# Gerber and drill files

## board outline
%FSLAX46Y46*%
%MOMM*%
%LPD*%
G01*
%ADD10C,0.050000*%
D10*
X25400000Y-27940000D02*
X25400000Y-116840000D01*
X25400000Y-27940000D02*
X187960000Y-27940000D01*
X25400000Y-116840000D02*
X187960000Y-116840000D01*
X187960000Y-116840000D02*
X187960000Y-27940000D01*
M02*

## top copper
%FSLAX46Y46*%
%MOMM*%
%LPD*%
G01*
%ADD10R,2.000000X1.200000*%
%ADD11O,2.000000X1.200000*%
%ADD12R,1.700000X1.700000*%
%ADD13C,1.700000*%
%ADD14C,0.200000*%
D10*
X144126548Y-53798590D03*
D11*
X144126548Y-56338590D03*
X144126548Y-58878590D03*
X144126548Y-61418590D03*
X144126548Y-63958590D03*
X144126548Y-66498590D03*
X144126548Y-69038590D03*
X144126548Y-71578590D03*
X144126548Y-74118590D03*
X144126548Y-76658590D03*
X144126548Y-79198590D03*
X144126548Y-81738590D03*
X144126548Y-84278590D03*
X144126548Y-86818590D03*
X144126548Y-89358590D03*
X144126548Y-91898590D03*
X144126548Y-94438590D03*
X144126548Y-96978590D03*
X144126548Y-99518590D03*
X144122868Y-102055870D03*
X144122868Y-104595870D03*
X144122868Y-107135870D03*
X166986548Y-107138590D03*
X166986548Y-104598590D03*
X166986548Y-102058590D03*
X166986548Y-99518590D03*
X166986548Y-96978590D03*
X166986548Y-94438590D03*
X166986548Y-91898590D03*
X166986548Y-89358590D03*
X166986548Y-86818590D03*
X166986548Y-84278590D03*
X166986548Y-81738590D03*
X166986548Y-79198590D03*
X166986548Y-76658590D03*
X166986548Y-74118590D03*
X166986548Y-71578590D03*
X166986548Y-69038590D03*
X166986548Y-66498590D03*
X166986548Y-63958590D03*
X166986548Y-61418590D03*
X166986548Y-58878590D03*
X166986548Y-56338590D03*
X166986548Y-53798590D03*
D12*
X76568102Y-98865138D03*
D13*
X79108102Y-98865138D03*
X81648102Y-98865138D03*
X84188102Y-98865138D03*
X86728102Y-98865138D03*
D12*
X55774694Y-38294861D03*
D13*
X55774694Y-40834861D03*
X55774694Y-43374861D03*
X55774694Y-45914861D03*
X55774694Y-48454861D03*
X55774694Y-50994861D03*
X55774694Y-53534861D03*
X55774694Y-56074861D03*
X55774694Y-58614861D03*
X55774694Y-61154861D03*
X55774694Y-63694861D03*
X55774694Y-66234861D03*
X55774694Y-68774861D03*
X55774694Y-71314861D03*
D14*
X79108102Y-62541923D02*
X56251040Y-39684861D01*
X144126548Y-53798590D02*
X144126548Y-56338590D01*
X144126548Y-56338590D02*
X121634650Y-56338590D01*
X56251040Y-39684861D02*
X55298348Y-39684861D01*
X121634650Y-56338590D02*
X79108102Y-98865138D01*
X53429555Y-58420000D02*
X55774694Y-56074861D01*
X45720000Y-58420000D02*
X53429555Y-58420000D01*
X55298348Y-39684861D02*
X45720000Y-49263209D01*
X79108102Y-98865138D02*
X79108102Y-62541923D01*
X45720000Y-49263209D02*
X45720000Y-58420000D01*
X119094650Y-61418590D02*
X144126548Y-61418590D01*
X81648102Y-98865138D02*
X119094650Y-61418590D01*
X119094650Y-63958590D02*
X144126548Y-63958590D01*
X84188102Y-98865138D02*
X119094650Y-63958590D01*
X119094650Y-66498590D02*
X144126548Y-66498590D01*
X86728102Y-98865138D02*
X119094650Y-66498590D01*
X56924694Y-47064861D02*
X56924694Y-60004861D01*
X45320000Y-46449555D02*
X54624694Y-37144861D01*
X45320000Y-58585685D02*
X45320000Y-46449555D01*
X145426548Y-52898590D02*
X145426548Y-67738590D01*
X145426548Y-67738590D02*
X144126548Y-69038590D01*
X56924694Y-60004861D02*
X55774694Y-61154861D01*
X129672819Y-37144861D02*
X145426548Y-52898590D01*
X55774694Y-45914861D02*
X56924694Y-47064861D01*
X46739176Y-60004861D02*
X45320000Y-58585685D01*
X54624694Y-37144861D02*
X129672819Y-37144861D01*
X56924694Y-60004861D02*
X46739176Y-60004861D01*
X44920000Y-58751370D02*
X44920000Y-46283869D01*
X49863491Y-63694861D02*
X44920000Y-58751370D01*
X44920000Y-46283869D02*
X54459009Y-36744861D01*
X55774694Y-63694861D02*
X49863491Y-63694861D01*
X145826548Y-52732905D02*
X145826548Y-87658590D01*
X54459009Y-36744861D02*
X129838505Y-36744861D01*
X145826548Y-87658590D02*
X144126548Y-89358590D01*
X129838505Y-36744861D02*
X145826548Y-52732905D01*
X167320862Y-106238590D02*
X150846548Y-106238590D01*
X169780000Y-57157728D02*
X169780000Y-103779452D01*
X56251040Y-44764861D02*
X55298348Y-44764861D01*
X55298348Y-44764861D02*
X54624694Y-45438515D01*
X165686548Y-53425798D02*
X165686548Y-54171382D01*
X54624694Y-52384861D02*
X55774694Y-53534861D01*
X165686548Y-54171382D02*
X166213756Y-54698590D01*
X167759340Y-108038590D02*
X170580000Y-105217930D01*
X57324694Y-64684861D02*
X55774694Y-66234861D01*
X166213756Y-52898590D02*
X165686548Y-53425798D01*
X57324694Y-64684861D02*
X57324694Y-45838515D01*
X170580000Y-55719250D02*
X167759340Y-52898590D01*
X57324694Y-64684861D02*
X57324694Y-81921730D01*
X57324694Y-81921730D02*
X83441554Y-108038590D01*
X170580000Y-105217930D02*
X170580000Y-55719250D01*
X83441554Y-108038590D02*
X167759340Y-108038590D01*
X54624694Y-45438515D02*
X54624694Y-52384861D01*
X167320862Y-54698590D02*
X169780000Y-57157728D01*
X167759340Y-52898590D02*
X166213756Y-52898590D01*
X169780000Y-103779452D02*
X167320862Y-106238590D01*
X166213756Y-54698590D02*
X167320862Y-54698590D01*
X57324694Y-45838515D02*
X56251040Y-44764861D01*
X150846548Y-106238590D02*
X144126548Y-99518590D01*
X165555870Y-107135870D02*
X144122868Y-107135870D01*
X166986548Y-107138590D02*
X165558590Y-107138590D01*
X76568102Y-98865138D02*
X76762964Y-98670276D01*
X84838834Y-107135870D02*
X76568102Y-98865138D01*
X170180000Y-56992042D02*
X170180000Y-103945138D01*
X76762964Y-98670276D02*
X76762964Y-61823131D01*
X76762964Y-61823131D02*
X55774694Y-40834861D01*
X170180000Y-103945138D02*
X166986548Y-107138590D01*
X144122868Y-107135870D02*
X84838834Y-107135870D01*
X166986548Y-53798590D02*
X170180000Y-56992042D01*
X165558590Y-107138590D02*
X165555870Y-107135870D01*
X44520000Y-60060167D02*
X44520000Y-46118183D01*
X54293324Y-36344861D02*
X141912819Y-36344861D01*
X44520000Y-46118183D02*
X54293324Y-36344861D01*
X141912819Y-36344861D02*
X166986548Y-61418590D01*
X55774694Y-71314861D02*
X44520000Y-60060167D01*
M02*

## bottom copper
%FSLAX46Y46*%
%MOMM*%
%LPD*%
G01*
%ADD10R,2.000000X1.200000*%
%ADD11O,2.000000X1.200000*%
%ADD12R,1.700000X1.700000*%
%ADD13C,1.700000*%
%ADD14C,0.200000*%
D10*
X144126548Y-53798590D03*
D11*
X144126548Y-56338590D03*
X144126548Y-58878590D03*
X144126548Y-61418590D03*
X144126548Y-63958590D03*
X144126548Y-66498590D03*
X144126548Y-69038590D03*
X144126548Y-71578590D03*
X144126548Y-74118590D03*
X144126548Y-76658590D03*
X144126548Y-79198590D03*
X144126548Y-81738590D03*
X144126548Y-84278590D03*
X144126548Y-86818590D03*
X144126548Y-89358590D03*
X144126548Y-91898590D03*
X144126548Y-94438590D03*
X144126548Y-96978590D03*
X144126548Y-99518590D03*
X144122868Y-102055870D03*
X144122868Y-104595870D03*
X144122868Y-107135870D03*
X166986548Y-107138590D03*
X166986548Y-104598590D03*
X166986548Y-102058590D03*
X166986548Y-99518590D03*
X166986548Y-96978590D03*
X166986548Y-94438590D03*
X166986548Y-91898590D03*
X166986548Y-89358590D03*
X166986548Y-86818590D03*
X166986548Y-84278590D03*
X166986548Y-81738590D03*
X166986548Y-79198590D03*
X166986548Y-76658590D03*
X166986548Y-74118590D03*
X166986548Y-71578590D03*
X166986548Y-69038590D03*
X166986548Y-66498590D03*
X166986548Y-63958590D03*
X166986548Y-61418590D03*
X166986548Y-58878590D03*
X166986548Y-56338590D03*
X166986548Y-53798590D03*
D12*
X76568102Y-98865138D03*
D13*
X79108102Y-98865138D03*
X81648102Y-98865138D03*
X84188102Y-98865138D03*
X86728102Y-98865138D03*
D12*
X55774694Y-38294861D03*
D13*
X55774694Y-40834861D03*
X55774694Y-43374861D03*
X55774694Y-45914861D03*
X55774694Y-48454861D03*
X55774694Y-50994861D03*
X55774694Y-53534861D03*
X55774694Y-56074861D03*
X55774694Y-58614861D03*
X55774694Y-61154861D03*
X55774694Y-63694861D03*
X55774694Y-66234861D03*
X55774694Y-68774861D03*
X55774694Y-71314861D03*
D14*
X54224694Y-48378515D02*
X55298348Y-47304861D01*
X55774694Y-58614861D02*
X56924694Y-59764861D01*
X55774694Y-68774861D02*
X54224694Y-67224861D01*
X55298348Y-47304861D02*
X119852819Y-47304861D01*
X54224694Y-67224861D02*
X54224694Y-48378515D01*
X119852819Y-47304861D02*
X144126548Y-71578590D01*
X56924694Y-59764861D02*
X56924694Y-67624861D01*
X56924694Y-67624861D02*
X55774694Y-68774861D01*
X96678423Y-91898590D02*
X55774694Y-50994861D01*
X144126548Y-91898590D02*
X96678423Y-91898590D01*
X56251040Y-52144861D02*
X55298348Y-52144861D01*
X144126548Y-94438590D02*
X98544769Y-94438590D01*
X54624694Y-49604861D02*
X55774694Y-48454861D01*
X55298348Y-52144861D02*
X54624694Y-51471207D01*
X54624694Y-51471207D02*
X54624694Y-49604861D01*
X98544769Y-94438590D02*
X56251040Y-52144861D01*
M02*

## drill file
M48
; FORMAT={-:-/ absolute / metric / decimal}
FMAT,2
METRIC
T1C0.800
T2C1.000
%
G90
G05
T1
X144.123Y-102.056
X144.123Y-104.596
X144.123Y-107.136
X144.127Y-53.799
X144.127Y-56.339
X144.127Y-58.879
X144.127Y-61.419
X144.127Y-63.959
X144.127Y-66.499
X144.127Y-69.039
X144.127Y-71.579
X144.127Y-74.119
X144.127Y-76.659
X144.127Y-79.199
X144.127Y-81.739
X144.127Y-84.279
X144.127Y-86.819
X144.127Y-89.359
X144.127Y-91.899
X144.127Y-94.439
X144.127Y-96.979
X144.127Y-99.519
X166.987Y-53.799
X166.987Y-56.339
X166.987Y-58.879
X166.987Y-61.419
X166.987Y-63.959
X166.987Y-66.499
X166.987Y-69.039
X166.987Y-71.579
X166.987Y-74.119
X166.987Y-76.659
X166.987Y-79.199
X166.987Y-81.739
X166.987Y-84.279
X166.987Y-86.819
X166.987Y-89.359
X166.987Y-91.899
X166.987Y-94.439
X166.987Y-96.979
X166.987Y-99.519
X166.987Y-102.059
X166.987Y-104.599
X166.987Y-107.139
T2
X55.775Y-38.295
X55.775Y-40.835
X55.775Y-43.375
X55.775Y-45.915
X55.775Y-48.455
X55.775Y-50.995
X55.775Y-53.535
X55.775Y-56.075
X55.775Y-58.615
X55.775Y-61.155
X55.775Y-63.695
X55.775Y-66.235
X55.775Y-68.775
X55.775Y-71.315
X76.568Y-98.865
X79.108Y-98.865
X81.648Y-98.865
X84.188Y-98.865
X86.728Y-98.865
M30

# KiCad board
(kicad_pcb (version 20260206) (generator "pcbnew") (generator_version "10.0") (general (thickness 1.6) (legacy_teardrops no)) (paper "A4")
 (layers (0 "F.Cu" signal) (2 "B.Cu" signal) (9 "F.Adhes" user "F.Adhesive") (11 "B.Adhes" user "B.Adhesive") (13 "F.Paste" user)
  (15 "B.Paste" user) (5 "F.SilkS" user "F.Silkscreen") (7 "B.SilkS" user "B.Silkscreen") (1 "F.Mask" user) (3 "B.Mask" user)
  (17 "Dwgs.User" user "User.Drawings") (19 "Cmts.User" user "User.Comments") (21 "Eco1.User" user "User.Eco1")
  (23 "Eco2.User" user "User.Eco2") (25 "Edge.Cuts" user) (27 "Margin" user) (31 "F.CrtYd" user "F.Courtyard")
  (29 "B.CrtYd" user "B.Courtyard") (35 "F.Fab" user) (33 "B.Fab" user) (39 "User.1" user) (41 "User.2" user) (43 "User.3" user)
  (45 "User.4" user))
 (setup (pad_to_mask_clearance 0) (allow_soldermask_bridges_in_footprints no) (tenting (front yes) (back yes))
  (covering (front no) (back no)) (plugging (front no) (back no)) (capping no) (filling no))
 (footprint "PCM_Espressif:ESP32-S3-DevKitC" (layer "F.Cu") (at 144.126548 53.79859)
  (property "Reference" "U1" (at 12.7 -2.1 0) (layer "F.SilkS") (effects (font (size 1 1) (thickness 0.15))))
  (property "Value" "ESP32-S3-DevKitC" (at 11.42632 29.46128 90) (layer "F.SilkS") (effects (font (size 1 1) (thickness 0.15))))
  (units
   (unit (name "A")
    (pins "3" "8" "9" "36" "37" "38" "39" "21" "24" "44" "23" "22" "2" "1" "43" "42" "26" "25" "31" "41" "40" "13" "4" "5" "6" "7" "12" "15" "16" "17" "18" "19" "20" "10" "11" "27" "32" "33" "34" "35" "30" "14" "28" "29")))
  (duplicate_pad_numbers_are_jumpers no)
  (pad "1" thru_hole rect (at 0 0 270) (size 1.2 2) (drill 0.8) (layers "*.Cu" "*.Mask") (remove_unused_layers no) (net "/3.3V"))
  (pad "2" thru_hole oval (at 0 2.54 270) (size 1.2 2) (drill 0.8) (layers "*.Cu" "*.Mask") (remove_unused_layers no) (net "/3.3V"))
  (pad "3" thru_hole oval (at 0 5.08 270) (size 1.2 2) (drill 0.8) (layers "*.Cu" "*.Mask") (remove_unused_layers no)
   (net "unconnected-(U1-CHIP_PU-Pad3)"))
  (pad "4" thru_hole oval (at 0 7.62 270) (size 1.2 2) (drill 0.8) (layers "*.Cu" "*.Mask") (remove_unused_layers no) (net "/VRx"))
  (pad "5" thru_hole oval (at 0 10.16 270) (size 1.2 2) (drill 0.8) (layers "*.Cu" "*.Mask") (remove_unused_layers no) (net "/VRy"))
  (pad "6" thru_hole oval (at 0 12.7 270) (size 1.2 2) (drill 0.8) (layers "*.Cu" "*.Mask") (remove_unused_layers no) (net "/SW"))
  (pad "7" thru_hole oval (at 0 15.24 270) (size 1.2 2) (drill 0.8) (layers "*.Cu" "*.Mask") (remove_unused_layers no) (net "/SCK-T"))
  (pad "8" thru_hole oval (at 0 17.78 270) (size 1.2 2) (drill 0.8) (layers "*.Cu" "*.Mask") (remove_unused_layers no) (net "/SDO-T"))
  (pad "9" thru_hole oval (at 0 20.32 270) (size 1.2 2) (drill 0.8) (layers "*.Cu" "*.Mask") (remove_unused_layers no)
   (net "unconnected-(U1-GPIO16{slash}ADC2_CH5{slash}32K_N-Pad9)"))
  (pad "10" thru_hole oval (at 0 22.86 270) (size 1.2 2) (drill 0.8) (layers "*.Cu" "*.Mask") (remove_unused_layers no)
   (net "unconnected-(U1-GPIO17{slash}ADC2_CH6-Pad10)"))
  (pad "11" thru_hole oval (at 0 25.4 270) (size 1.2 2) (drill 0.8) (layers "*.Cu" "*.Mask") (remove_unused_layers no)
   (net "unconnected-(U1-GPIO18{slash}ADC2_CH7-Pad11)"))
  (pad "12" thru_hole oval (at 0 27.94 270) (size 1.2 2) (drill 0.8) (layers "*.Cu" "*.Mask") (remove_unused_layers no)
   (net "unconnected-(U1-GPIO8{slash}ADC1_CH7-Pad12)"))
  (pad "13" thru_hole oval (at 0 30.48 270) (size 1.2 2) (drill 0.8) (layers "*.Cu" "*.Mask") (remove_unused_layers no)
   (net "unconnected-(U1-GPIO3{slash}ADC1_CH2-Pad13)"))
  (pad "14" thru_hole oval (at 0 33.02 270) (size 1.2 2) (drill 0.8) (layers "*.Cu" "*.Mask") (remove_unused_layers no)
   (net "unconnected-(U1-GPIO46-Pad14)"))
  (pad "15" thru_hole oval (at 0 35.56 270) (size 1.2 2) (drill 0.8) (layers "*.Cu" "*.Mask") (remove_unused_layers no) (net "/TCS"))
  (pad "16" thru_hole oval (at 0 38.1 270) (size 1.2 2) (drill 0.8) (layers "*.Cu" "*.Mask") (remove_unused_layers no) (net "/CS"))
  (pad "17" thru_hole oval (at 0 40.64 270) (size 1.2 2) (drill 0.8) (layers "*.Cu" "*.Mask") (remove_unused_layers no) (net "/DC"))
  (pad "18" thru_hole oval (at 0 43.18 270) (size 1.2 2) (drill 0.8) (layers "*.Cu" "*.Mask") (remove_unused_layers no)
   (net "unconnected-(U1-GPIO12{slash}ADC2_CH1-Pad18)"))
  (pad "19" thru_hole oval (at 0 45.72 270) (size 1.2 2) (drill 0.8) (layers "*.Cu" "*.Mask") (remove_unused_layers no) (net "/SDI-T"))
  (pad "20" thru_hole oval (at -0.00368 48.25728 270) (size 1.2 2) (drill 0.8) (layers "*.Cu" "*.Mask") (remove_unused_layers no)
   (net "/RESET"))
  (pad "21" thru_hole oval (at -0.00368 50.79728 270) (size 1.2 2) (drill 0.8) (layers "*.Cu" "*.Mask") (remove_unused_layers no)
   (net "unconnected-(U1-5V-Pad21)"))
  (pad "22" thru_hole oval (at -0.00368 53.33728 270) (size 1.2 2) (drill 0.8) (layers "*.Cu" "*.Mask") (remove_unused_layers no)
   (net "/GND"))
  (pad "23" thru_hole oval (at 22.86 53.34 270) (size 1.2 2) (drill 0.8) (layers "*.Cu" "*.Mask") (remove_unused_layers no) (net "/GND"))
  (pad "24" thru_hole oval (at 22.86 50.8 270) (size 1.2 2) (drill 0.8) (layers "*.Cu" "*.Mask") (remove_unused_layers no) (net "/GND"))
  (pad "25" thru_hole oval (at 22.86 48.26 270) (size 1.2 2) (drill 0.8) (layers "*.Cu" "*.Mask") (remove_unused_layers no)
   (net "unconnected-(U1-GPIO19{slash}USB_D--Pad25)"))
  (pad "26" thru_hole oval (at 22.86 45.72 270) (size 1.2 2) (drill 0.8) (layers "*.Cu" "*.Mask") (remove_unused_layers no)
   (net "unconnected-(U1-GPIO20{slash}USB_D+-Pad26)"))
  (pad "27" thru_hole oval (at 22.86 43.18 270) (size 1.2 2) (drill 0.8) (layers "*.Cu" "*.Mask") (remove_unused_layers no)
   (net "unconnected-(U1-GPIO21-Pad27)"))
  (pad "28" thru_hole oval (at 22.86 40.64 270) (size 1.2 2) (drill 0.8) (layers "*.Cu" "*.Mask") (remove_unused_layers no)
   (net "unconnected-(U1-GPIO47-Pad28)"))
  (pad "29" thru_hole oval (at 22.86 38.1 270) (size 1.2 2) (drill 0.8) (layers "*.Cu" "*.Mask") (remove_unused_layers no)
   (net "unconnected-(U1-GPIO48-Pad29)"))
  (pad "30" thru_hole oval (at 22.86 35.56 270) (size 1.2 2) (drill 0.8) (layers "*.Cu" "*.Mask") (remove_unused_layers no)
   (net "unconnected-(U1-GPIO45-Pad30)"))
  (pad "31" thru_hole oval (at 22.86 33.02 270) (size 1.2 2) (drill 0.8) (layers "*.Cu" "*.Mask") (remove_unused_layers no)
   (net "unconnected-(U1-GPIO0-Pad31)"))
  (pad "32" thru_hole oval (at 22.86 30.48 270) (size 1.2 2) (drill 0.8) (layers "*.Cu" "*.Mask") (remove_unused_layers no)
   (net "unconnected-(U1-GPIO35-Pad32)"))
  (pad "33" thru_hole oval (at 22.86 27.94 270) (size 1.2 2) (drill 0.8) (layers "*.Cu" "*.Mask") (remove_unused_layers no)
   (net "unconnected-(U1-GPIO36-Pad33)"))
  (pad "34" thru_hole oval (at 22.86 25.4 270) (size 1.2 2) (drill 0.8) (layers "*.Cu" "*.Mask") (remove_unused_layers no)
   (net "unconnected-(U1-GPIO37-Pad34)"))
  (pad "35" thru_hole oval (at 22.86 22.86 270) (size 1.2 2) (drill 0.8) (layers "*.Cu" "*.Mask") (remove_unused_layers no)
   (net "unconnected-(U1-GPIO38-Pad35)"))
  (pad "36" thru_hole oval (at 22.86 20.32 270) (size 1.2 2) (drill 0.8) (layers "*.Cu" "*.Mask") (remove_unused_layers no)
   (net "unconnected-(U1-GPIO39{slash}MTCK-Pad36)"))
  (pad "37" thru_hole oval (at 22.86 17.78 270) (size 1.2 2) (drill 0.8) (layers "*.Cu" "*.Mask") (remove_unused_layers no)
   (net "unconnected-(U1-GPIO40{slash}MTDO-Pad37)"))
  (pad "38" thru_hole oval (at 22.86 15.24 270) (size 1.2 2) (drill 0.8) (layers "*.Cu" "*.Mask") (remove_unused_layers no)
   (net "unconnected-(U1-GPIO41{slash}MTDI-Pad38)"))
  (pad "39" thru_hole oval (at 22.86 12.7 270) (size 1.2 2) (drill 0.8) (layers "*.Cu" "*.Mask") (remove_unused_layers no)
   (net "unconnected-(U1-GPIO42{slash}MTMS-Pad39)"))
  (pad "40" thru_hole oval (at 22.86 10.16 270) (size 1.2 2) (drill 0.8) (layers "*.Cu" "*.Mask") (remove_unused_layers no)
   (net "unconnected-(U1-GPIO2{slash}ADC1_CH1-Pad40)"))
  (pad "41" thru_hole oval (at 22.86 7.62 270) (size 1.2 2) (drill 0.8) (layers "*.Cu" "*.Mask") (remove_unused_layers no) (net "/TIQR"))
  (pad "42" thru_hole oval (at 22.86 5.08 270) (size 1.2 2) (drill 0.8) (layers "*.Cu" "*.Mask") (remove_unused_layers no)
   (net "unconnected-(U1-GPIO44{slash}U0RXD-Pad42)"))
  (pad "43" thru_hole oval (at 22.86 2.54 270) (size 1.2 2) (drill 0.8) (layers "*.Cu" "*.Mask") (remove_unused_layers no)
   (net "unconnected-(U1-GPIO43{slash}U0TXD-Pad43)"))
  (pad "44" thru_hole oval (at 22.86 0 270) (size 1.2 2) (drill 0.8) (layers "*.Cu" "*.Mask") (remove_unused_layers no) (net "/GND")))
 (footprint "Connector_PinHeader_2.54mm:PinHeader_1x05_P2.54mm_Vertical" (layer "F.Cu") (at 76.568102 98.865138 90)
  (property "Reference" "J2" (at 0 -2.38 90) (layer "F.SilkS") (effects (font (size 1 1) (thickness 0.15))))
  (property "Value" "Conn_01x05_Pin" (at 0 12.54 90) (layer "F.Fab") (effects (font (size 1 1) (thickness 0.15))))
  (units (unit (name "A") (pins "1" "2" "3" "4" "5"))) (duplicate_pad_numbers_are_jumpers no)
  (pad "1" thru_hole rect (at 0 0 90) (size 1.7 1.7) (drill 1) (layers "*.Cu" "*.Mask") (remove_unused_layers no) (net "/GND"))
  (pad "2" thru_hole circle (at 0 2.54 90) (size 1.7 1.7) (drill 1) (layers "*.Cu" "*.Mask") (remove_unused_layers no) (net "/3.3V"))
  (pad "3" thru_hole circle (at 0 5.08 90) (size 1.7 1.7) (drill 1) (layers "*.Cu" "*.Mask") (remove_unused_layers no) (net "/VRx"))
  (pad "4" thru_hole circle (at 0 7.62 90) (size 1.7 1.7) (drill 1) (layers "*.Cu" "*.Mask") (remove_unused_layers no) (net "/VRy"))
  (pad "5" thru_hole circle (at 0 10.16 90) (size 1.7 1.7) (drill 1) (layers "*.Cu" "*.Mask") (remove_unused_layers no) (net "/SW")))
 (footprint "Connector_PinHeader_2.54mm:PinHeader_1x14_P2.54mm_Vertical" (layer "F.Cu") (at 55.774694 38.294861)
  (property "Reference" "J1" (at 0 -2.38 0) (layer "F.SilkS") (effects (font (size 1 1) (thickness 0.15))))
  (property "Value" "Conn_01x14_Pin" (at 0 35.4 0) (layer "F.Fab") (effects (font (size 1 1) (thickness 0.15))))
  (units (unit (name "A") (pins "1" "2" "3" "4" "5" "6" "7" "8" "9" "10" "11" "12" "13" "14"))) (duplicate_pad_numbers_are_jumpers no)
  (pad "1" thru_hole rect (at 0 0) (size 1.7 1.7) (drill 1) (layers "*.Cu" "*.Mask") (remove_unused_layers no) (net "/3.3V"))
  (pad "2" thru_hole circle (at 0 2.54) (size 1.7 1.7) (drill 1) (layers "*.Cu" "*.Mask") (remove_unused_layers no) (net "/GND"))
  (pad "3" thru_hole circle (at 0 5.08) (size 1.7 1.7) (drill 1) (layers "*.Cu" "*.Mask") (remove_unused_layers no) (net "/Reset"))
  (pad "4" thru_hole circle (at 0 7.62) (size 1.7 1.7) (drill 1) (layers "*.Cu" "*.Mask") (remove_unused_layers no) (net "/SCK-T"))
  (pad "5" thru_hole circle (at 0 10.16) (size 1.7 1.7) (drill 1) (layers "*.Cu" "*.Mask") (remove_unused_layers no) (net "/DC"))
  (pad "6" thru_hole circle (at 0 12.7) (size 1.7 1.7) (drill 1) (layers "*.Cu" "*.Mask") (remove_unused_layers no) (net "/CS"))
  (pad "7" thru_hole circle (at 0 15.24) (size 1.7 1.7) (drill 1) (layers "*.Cu" "*.Mask") (remove_unused_layers no) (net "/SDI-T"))
  (pad "8" thru_hole circle (at 0 17.78) (size 1.7 1.7) (drill 1) (layers "*.Cu" "*.Mask") (remove_unused_layers no) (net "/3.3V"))
  (pad "9" thru_hole circle (at 0 20.32) (size 1.7 1.7) (drill 1) (layers "*.Cu" "*.Mask") (remove_unused_layers no) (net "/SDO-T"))
  (pad "10" thru_hole circle (at 0 22.86) (size 1.7 1.7) (drill 1) (layers "*.Cu" "*.Mask") (remove_unused_layers no) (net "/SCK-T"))
  (pad "11" thru_hole circle (at 0 25.4) (size 1.7 1.7) (drill 1) (layers "*.Cu" "*.Mask") (remove_unused_layers no) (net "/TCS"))
  (pad "12" thru_hole circle (at 0 27.94) (size 1.7 1.7) (drill 1) (layers "*.Cu" "*.Mask") (remove_unused_layers no) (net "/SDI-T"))
  (pad "13" thru_hole circle (at 0 30.48) (size 1.7 1.7) (drill 1) (layers "*.Cu" "*.Mask") (remove_unused_layers no) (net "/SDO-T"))
  (pad "14" thru_hole circle (at 0 33.02) (size 1.7 1.7) (drill 1) (layers "*.Cu" "*.Mask") (remove_unused_layers no) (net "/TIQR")))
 (gr_line (start 25.4 27.94) (end 25.4 116.84) (stroke (width 0.05) (type default)) (layer "Edge.Cuts"))
 (gr_line (start 25.4 27.94) (end 187.96 27.94) (stroke (width 0.05) (type default)) (layer "Edge.Cuts"))
 (gr_line (start 25.4 116.84) (end 187.96 116.84) (stroke (width 0.05) (type default)) (layer "Edge.Cuts"))
 (gr_line (start 187.96 116.84) (end 187.96 27.94) (stroke (width 0.05) (type default)) (layer "Edge.Cuts"))
 (segment (start 79.108102 62.541923) (end 56.25104 39.684861) (width 0.2) (layer "F.Cu") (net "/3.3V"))
 (segment (start 144.126548 53.79859) (end 144.126548 56.33859) (width 0.2) (layer "F.Cu") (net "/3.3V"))
 (segment (start 144.126548 56.33859) (end 121.63465 56.33859) (width 0.2) (layer "F.Cu") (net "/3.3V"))
 (segment (start 56.25104 39.684861) (end 55.298348 39.684861) (width 0.2) (layer "F.Cu") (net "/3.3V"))
 (segment (start 121.63465 56.33859) (end 79.108102 98.865138) (width 0.2) (layer "F.Cu") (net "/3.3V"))
 (segment (start 53.429555 58.42) (end 55.774694 56.074861) (width 0.2) (layer "F.Cu") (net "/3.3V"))
 (segment (start 45.72 58.42) (end 53.429555 58.42) (width 0.2) (layer "F.Cu") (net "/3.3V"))
 (segment (start 55.298348 39.684861) (end 45.72 49.263209) (width 0.2) (layer "F.Cu") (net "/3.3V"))
 (segment (start 79.108102 98.865138) (end 79.108102 62.541923) (width 0.2) (layer "F.Cu") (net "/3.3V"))
 (segment (start 45.72 49.263209) (end 45.72 58.42) (width 0.2) (layer "F.Cu") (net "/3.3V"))
 (segment (start 119.09465 61.41859) (end 144.126548 61.41859) (width 0.2) (layer "F.Cu") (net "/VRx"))
 (segment (start 81.648102 98.865138) (end 119.09465 61.41859) (width 0.2) (layer "F.Cu") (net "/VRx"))
 (segment (start 119.09465 63.95859) (end 144.126548 63.95859) (width 0.2) (layer "F.Cu") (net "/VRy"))
 (segment (start 84.188102 98.865138) (end 119.09465 63.95859) (width 0.2) (layer "F.Cu") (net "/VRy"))
 (segment (start 119.09465 66.49859) (end 144.126548 66.49859) (width 0.2) (layer "F.Cu") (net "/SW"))
 (segment (start 86.728102 98.865138) (end 119.09465 66.49859) (width 0.2) (layer "F.Cu") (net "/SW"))
 (segment (start 56.924694 47.064861) (end 56.924694 60.004861) (width 0.2) (layer "F.Cu") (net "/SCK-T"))
 (segment (start 45.32 46.449555) (end 54.624694 37.144861) (width 0.2) (layer "F.Cu") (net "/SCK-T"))
 (segment (start 45.32 58.585685) (end 45.32 46.449555) (width 0.2) (layer "F.Cu") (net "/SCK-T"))
 (segment (start 145.426548 52.89859) (end 145.426548 67.73859) (width 0.2) (layer "F.Cu") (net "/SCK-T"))
 (segment (start 145.426548 67.73859) (end 144.126548 69.03859) (width 0.2) (layer "F.Cu") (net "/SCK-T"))
 (segment (start 56.924694 60.004861) (end 55.774694 61.154861) (width 0.2) (layer "F.Cu") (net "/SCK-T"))
 (segment (start 129.672819 37.144861) (end 145.426548 52.89859) (width 0.2) (layer "F.Cu") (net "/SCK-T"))
 (segment (start 55.774694 45.914861) (end 56.924694 47.064861) (width 0.2) (layer "F.Cu") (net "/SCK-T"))
 (segment (start 46.739176 60.004861) (end 45.32 58.585685) (width 0.2) (layer "F.Cu") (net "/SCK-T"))
 (segment (start 54.624694 37.144861) (end 129.672819 37.144861) (width 0.2) (layer "F.Cu") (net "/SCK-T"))
 (segment (start 56.924694 60.004861) (end 46.739176 60.004861) (width 0.2) (layer "F.Cu") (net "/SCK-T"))
 (segment (start 54.224694 48.378515) (end 55.298348 47.304861) (width 0.2) (layer "B.Cu") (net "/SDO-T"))
 (segment (start 55.774694 58.614861) (end 56.924694 59.764861) (width 0.2) (layer "B.Cu") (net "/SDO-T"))
 (segment (start 55.774694 68.774861) (end 54.224694 67.224861) (width 0.2) (layer "B.Cu") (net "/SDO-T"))
 (segment (start 55.298348 47.304861) (end 119.852819 47.304861) (width 0.2) (layer "B.Cu") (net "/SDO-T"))
 (segment (start 54.224694 67.224861) (end 54.224694 48.378515) (width 0.2) (layer "B.Cu") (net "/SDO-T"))
 (segment (start 119.852819 47.304861) (end 144.126548 71.57859) (width 0.2) (layer "B.Cu") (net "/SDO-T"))
 (segment (start 56.924694 59.764861) (end 56.924694 67.624861) (width 0.2) (layer "B.Cu") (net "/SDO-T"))
 (segment (start 56.924694 67.624861) (end 55.774694 68.774861) (width 0.2) (layer "B.Cu") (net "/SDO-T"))
 (segment (start 44.92 58.75137) (end 44.92 46.283869) (width 0.2) (layer "F.Cu") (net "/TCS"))
 (segment (start 49.863491 63.694861) (end 44.92 58.75137) (width 0.2) (layer "F.Cu") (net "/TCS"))
 (segment (start 44.92 46.283869) (end 54.459009 36.744861) (width 0.2) (layer "F.Cu") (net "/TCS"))
 (segment (start 55.774694 63.694861) (end 49.863491 63.694861) (width 0.2) (layer "F.Cu") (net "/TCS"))
 (segment (start 145.826548 52.732905) (end 145.826548 87.65859) (width 0.2) (layer "F.Cu") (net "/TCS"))
 (segment (start 54.459009 36.744861) (end 129.838505 36.744861) (width 0.2) (layer "F.Cu") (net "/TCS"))
 (segment (start 145.826548 87.65859) (end 144.126548 89.35859) (width 0.2) (layer "F.Cu") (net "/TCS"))
 (segment (start 129.838505 36.744861) (end 145.826548 52.732905) (width 0.2) (layer "F.Cu") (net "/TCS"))
 (segment (start 96.678423 91.89859) (end 55.774694 50.994861) (width 0.2) (layer "B.Cu") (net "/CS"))
 (segment (start 144.126548 91.89859) (end 96.678423 91.89859) (width 0.2) (layer "B.Cu") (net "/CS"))
 (segment (start 56.25104 52.144861) (end 55.298348 52.144861) (width 0.2) (layer "B.Cu") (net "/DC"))
 (segment (start 144.126548 94.43859) (end 98.544769 94.43859) (width 0.2) (layer "B.Cu") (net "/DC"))
 (segment (start 54.624694 49.604861) (end 55.774694 48.454861) (width 0.2) (layer "B.Cu") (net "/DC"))
 (segment (start 55.298348 52.144861) (end 54.624694 51.471207) (width 0.2) (layer "B.Cu") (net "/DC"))
 (segment (start 54.624694 51.471207) (end 54.624694 49.604861) (width 0.2) (layer "B.Cu") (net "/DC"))
 (segment (start 98.544769 94.43859) (end 56.25104 52.144861) (width 0.2) (layer "B.Cu") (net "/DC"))
 (segment (start 167.320862 106.23859) (end 150.846548 106.23859) (width 0.2) (layer "F.Cu") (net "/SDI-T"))
 (segment (start 169.78 57.157728) (end 169.78 103.779452) (width 0.2) (layer "F.Cu") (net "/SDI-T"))
 (segment (start 56.25104 44.764861) (end 55.298348 44.764861) (width 0.2) (layer "F.Cu") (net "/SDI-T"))
 (segment (start 55.298348 44.764861) (end 54.624694 45.438515) (width 0.2) (layer "F.Cu") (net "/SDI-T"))
 (segment (start 165.686548 53.425798) (end 165.686548 54.171382) (width 0.2) (layer "F.Cu") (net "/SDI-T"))
 (segment (start 54.624694 52.384861) (end 55.774694 53.534861) (width 0.2) (layer "F.Cu") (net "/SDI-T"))
 (segment (start 165.686548 54.171382) (end 166.213756 54.69859) (width 0.2) (layer "F.Cu") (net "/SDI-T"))
 (segment (start 167.75934 108.03859) (end 170.58 105.21793) (width 0.2) (layer "F.Cu") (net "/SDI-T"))
 (segment (start 57.324694 64.684861) (end 55.774694 66.234861) (width 0.2) (layer "F.Cu") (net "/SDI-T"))
 (segment (start 166.213756 52.89859) (end 165.686548 53.425798) (width 0.2) (layer "F.Cu") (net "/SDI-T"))
 (segment (start 57.324694 64.684861) (end 57.324694 45.838515) (width 0.2) (layer "F.Cu") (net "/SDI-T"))
 (segment (start 170.58 55.71925) (end 167.75934 52.89859) (width 0.2) (layer "F.Cu") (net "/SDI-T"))
 (segment (start 57.324694 64.684861) (end 57.324694 81.92173) (width 0.2) (layer "F.Cu") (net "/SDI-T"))
 (segment (start 57.324694 81.92173) (end 83.441554 108.03859) (width 0.2) (layer "F.Cu") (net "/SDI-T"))
 (segment (start 170.58 105.21793) (end 170.58 55.71925) (width 0.2) (layer "F.Cu") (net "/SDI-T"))
 (segment (start 83.441554 108.03859) (end 167.75934 108.03859) (width 0.2) (layer "F.Cu") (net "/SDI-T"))
 (segment (start 54.624694 45.438515) (end 54.624694 52.384861) (width 0.2) (layer "F.Cu") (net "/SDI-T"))
 (segment (start 167.320862 54.69859) (end 169.78 57.157728) (width 0.2) (layer "F.Cu") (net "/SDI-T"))
 (segment (start 167.75934 52.89859) (end 166.213756 52.89859) (width 0.2) (layer "F.Cu") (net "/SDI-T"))
 (segment (start 169.78 103.779452) (end 167.320862 106.23859) (width 0.2) (layer "F.Cu") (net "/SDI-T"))
 (segment (start 166.213756 54.69859) (end 167.320862 54.69859) (width 0.2) (layer "F.Cu") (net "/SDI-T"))
 (segment (start 57.324694 45.838515) (end 56.25104 44.764861) (width 0.2) (layer "F.Cu") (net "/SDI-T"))
 (segment (start 150.846548 106.23859) (end 144.126548 99.51859) (width 0.2) (layer "F.Cu") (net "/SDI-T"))
 (segment (start 165.55587 107.13587) (end 144.122868 107.13587) (width 0.2) (layer "F.Cu") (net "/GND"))
 (segment (start 166.986548 107.13859) (end 165.55859 107.13859) (width 0.2) (layer "F.Cu") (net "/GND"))
 (segment (start 76.568102 98.865138) (end 76.762964 98.670276) (width 0.2) (layer "F.Cu") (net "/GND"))
 (segment (start 84.838834 107.13587) (end 76.568102 98.865138) (width 0.2) (layer "F.Cu") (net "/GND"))
 (segment (start 170.18 56.992042) (end 170.18 103.945138) (width 0.2) (layer "F.Cu") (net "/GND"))
 (segment (start 76.762964 98.670276) (end 76.762964 61.823131) (width 0.2) (layer "F.Cu") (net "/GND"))
 (segment (start 76.762964 61.823131) (end 55.774694 40.834861) (width 0.2) (layer "F.Cu") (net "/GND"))
 (segment (start 170.18 103.945138) (end 166.986548 107.13859) (width 0.2) (layer "F.Cu") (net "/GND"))
 (segment (start 144.122868 107.13587) (end 84.838834 107.13587) (width 0.2) (layer "F.Cu") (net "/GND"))
 (segment (start 166.986548 53.79859) (end 170.18 56.992042) (width 0.2) (layer "F.Cu") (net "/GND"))
 (segment (start 165.55859 107.13859) (end 165.55587 107.13587) (width 0.2) (layer "F.Cu") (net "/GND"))
 (segment (start 44.52 60.060167) (end 44.52 46.118183) (width 0.2) (layer "F.Cu") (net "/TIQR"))
 (segment (start 54.293324 36.344861) (end 141.912819 36.344861) (width 0.2) (layer "F.Cu") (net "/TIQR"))
 (segment (start 44.52 46.118183) (end 54.293324 36.344861) (width 0.2) (layer "F.Cu") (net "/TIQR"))
 (segment (start 141.912819 36.344861) (end 166.986548 61.41859) (width 0.2) (layer "F.Cu") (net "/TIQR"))
 (segment (start 55.774694 71.314861) (end 44.52 60.060167) (width 0.2) (layer "F.Cu") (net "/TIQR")))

